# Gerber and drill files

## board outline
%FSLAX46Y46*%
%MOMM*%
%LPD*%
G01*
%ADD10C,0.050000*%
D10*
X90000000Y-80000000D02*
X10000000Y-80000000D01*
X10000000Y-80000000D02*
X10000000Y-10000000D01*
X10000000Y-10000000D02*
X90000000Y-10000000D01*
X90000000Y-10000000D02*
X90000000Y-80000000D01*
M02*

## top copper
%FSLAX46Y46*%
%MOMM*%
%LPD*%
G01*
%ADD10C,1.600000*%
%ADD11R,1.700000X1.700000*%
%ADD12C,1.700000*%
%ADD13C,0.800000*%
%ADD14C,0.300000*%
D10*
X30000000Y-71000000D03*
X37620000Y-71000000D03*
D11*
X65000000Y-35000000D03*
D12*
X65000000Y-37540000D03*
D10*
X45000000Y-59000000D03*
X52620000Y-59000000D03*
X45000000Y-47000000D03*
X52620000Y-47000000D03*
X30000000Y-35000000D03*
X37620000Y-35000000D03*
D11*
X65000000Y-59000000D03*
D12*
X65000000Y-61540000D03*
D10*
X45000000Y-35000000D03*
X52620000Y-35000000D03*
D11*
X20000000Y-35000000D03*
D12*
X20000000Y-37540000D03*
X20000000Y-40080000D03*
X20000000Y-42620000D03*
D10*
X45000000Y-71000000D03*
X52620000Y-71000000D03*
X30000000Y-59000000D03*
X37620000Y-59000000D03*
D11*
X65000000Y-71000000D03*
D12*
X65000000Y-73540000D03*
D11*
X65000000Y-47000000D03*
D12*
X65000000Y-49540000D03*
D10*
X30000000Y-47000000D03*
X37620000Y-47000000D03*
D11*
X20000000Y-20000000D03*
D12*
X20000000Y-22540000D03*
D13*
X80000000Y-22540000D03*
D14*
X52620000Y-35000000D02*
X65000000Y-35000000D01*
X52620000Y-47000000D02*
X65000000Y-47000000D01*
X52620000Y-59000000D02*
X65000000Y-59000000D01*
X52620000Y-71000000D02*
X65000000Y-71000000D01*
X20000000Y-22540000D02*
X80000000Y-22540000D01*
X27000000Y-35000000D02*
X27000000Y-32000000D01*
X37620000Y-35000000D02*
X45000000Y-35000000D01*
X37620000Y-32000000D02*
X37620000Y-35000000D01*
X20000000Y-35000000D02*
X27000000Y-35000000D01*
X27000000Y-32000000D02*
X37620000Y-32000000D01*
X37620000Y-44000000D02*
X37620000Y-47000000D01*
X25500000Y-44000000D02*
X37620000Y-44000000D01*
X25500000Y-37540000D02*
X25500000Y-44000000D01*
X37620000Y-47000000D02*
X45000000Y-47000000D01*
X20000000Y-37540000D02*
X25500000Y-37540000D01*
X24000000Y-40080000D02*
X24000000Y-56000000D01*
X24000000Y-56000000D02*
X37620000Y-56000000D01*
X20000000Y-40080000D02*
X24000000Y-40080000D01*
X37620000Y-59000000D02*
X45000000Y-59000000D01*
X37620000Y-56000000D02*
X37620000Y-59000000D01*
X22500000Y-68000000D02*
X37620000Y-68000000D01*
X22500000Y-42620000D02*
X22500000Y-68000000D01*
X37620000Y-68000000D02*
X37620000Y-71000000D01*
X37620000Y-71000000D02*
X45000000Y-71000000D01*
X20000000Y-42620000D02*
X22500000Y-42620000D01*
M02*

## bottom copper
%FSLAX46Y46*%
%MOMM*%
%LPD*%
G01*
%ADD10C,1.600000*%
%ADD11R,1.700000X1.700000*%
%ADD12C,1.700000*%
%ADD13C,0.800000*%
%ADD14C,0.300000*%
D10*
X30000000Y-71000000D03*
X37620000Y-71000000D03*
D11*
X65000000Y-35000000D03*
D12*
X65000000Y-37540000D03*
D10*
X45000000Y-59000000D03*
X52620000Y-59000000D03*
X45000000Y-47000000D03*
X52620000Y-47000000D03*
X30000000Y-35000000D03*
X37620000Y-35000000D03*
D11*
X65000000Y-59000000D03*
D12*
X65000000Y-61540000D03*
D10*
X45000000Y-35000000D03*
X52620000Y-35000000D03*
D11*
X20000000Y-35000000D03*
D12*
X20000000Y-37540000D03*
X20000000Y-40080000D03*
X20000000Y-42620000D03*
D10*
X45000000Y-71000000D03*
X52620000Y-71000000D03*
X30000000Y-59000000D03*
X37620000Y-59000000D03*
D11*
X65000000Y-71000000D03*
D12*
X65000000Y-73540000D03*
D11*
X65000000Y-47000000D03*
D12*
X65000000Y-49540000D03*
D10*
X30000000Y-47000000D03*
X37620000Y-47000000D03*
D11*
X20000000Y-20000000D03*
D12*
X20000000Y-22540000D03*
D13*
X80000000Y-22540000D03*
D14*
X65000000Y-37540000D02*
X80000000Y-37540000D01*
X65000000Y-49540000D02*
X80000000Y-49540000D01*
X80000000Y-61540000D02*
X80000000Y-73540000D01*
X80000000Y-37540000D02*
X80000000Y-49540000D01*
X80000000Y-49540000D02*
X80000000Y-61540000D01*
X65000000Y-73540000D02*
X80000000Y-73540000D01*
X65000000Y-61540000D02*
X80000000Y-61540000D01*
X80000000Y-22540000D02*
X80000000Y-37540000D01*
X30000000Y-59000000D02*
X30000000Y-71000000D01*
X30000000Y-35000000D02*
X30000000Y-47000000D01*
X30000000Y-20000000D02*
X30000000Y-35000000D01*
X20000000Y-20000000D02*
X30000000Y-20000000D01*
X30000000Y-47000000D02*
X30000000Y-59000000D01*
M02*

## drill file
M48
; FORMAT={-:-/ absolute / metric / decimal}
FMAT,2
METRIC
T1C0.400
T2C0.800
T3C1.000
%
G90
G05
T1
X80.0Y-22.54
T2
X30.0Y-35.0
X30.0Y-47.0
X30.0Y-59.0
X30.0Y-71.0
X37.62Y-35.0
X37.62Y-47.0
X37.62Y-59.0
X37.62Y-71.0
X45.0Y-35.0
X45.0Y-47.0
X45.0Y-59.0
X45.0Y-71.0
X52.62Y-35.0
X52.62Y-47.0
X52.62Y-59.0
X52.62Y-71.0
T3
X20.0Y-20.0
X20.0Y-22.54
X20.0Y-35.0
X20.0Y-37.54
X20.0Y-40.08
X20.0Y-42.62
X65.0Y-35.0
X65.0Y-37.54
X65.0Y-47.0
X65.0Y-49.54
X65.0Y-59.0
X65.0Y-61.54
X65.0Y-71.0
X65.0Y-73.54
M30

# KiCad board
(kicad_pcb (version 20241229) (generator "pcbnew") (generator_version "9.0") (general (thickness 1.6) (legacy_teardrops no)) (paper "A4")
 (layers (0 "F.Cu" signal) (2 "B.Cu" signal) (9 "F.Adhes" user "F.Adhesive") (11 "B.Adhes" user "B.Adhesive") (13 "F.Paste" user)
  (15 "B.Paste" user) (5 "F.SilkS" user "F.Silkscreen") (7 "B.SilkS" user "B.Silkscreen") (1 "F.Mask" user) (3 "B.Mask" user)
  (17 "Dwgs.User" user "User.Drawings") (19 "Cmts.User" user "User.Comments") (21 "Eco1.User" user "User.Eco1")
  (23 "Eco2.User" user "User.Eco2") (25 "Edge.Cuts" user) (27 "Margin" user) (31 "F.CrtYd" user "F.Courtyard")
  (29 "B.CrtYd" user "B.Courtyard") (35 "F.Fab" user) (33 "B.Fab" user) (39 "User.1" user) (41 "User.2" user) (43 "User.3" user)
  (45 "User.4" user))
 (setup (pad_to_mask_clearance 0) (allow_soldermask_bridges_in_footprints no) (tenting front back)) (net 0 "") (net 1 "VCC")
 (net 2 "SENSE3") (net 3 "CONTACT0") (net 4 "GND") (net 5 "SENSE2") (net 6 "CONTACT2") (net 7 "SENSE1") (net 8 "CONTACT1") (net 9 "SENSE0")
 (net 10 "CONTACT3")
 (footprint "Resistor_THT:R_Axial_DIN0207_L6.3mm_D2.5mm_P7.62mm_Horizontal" (layer "F.Cu") (at 30 71)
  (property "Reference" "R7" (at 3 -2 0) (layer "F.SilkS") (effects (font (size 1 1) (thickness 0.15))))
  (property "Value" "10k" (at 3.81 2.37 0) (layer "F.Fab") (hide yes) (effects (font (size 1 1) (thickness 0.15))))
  (pad "1" thru_hole circle (at 0 0) (size 1.6 1.6) (drill 0.8) (layers "*.Cu" "*.Mask") (remove_unused_layers no) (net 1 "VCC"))
  (pad "2" thru_hole circle (at 7.62 0) (size 1.6 1.6) (drill 0.8) (layers "*.Cu" "*.Mask") (remove_unused_layers no) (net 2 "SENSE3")))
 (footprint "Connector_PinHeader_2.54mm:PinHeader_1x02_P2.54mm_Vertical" (layer "F.Cu") (at 65 35)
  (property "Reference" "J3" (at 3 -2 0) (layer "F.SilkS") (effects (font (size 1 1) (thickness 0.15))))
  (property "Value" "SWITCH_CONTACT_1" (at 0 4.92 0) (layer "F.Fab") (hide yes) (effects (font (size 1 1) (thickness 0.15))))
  (pad "1" thru_hole rect (at 0 0) (size 1.7 1.7) (drill 1) (layers "*.Cu" "*.Mask") (remove_unused_layers no) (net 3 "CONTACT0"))
  (pad "2" thru_hole circle (at 0 2.54) (size 1.7 1.7) (drill 1) (layers "*.Cu" "*.Mask") (remove_unused_layers no) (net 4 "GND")))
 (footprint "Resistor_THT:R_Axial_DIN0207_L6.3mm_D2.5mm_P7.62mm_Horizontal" (layer "F.Cu") (at 45 59)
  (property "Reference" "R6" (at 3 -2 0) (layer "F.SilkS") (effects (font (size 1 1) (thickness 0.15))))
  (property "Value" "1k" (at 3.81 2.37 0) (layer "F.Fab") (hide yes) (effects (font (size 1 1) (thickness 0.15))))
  (pad "1" thru_hole circle (at 0 0) (size 1.6 1.6) (drill 0.8) (layers "*.Cu" "*.Mask") (remove_unused_layers no) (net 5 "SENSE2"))
  (pad "2" thru_hole circle (at 7.62 0) (size 1.6 1.6) (drill 0.8) (layers "*.Cu" "*.Mask") (remove_unused_layers no) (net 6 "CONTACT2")))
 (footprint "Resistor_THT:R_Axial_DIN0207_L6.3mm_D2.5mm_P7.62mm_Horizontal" (layer "F.Cu") (at 45 47)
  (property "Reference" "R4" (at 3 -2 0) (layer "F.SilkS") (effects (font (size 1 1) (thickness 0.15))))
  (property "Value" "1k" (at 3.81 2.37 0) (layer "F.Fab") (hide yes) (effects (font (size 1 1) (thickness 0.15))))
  (pad "1" thru_hole circle (at 0 0) (size 1.6 1.6) (drill 0.8) (layers "*.Cu" "*.Mask") (remove_unused_layers no) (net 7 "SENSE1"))
  (pad "2" thru_hole circle (at 7.62 0) (size 1.6 1.6) (drill 0.8) (layers "*.Cu" "*.Mask") (remove_unused_layers no) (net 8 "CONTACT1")))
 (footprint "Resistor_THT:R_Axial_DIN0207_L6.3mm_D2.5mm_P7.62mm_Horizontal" (layer "F.Cu") (at 30 35)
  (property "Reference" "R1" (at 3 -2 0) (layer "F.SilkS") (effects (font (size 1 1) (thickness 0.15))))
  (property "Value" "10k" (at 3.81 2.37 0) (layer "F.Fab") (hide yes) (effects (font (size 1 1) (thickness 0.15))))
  (pad "1" thru_hole circle (at 0 0) (size 1.6 1.6) (drill 0.8) (layers "*.Cu" "*.Mask") (remove_unused_layers no) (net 1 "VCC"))
  (pad "2" thru_hole circle (at 7.62 0) (size 1.6 1.6) (drill 0.8) (layers "*.Cu" "*.Mask") (remove_unused_layers no) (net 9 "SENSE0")))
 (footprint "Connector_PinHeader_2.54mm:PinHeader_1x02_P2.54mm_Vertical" (layer "F.Cu") (at 65 59)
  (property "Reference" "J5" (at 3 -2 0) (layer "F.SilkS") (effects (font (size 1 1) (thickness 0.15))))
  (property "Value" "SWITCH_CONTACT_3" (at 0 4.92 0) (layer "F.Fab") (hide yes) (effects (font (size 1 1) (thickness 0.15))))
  (pad "1" thru_hole rect (at 0 0) (size 1.7 1.7) (drill 1) (layers "*.Cu" "*.Mask") (remove_unused_layers no) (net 6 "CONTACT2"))
  (pad "2" thru_hole circle (at 0 2.54) (size 1.7 1.7) (drill 1) (layers "*.Cu" "*.Mask") (remove_unused_layers no) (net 4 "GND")))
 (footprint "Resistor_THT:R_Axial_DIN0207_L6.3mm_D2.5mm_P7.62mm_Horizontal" (layer "F.Cu") (at 45 35)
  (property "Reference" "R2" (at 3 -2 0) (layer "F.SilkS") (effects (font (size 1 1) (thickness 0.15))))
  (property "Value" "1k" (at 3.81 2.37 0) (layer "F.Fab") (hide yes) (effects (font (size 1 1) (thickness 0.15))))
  (pad "1" thru_hole circle (at 0 0) (size 1.6 1.6) (drill 0.8) (layers "*.Cu" "*.Mask") (remove_unused_layers no) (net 9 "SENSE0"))
  (pad "2" thru_hole circle (at 7.62 0) (size 1.6 1.6) (drill 0.8) (layers "*.Cu" "*.Mask") (remove_unused_layers no) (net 3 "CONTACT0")))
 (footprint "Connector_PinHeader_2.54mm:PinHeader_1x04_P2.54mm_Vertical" (layer "F.Cu") (at 20 35)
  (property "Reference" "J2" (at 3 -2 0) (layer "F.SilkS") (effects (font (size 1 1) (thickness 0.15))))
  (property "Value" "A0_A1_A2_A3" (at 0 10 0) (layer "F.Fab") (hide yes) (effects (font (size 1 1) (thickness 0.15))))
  (pad "1" thru_hole rect (at 0 0) (size 1.7 1.7) (drill 1) (layers "*.Cu" "*.Mask") (remove_unused_layers no) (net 9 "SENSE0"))
  (pad "2" thru_hole circle (at 0 2.54) (size 1.7 1.7) (drill 1) (layers "*.Cu" "*.Mask") (remove_unused_layers no) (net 7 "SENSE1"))
  (pad "3" thru_hole circle (at 0 5.08) (size 1.7 1.7) (drill 1) (layers "*.Cu" "*.Mask") (remove_unused_layers no) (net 5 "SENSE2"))
  (pad "4" thru_hole circle (at 0 7.62) (size 1.7 1.7) (drill 1) (layers "*.Cu" "*.Mask") (remove_unused_layers no) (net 2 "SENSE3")))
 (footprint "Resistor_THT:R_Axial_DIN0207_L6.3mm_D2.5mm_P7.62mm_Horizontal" (layer "F.Cu") (at 45 71)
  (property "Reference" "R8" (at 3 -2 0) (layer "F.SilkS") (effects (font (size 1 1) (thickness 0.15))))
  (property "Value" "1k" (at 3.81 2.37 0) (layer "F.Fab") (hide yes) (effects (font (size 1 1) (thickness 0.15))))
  (pad "1" thru_hole circle (at 0 0) (size 1.6 1.6) (drill 0.8) (layers "*.Cu" "*.Mask") (remove_unused_layers no) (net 2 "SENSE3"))
  (pad "2" thru_hole circle (at 7.62 0) (size 1.6 1.6) (drill 0.8) (layers "*.Cu" "*.Mask") (remove_unused_layers no) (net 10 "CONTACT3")))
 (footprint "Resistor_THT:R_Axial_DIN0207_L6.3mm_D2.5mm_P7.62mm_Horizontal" (layer "F.Cu") (at 30 59)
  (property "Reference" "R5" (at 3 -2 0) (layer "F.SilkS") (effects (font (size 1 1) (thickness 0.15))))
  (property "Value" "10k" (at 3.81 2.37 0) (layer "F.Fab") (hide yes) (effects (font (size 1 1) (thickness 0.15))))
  (pad "1" thru_hole circle (at 0 0) (size 1.6 1.6) (drill 0.8) (layers "*.Cu" "*.Mask") (remove_unused_layers no) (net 1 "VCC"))
  (pad "2" thru_hole circle (at 7.62 0) (size 1.6 1.6) (drill 0.8) (layers "*.Cu" "*.Mask") (remove_unused_layers no) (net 5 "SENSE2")))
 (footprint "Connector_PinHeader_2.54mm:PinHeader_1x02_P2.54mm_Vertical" (layer "F.Cu") (at 65 71)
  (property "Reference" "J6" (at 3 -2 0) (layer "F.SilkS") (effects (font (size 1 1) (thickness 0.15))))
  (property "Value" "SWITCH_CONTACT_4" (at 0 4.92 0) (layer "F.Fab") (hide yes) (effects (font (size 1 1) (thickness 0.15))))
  (pad "1" thru_hole rect (at 0 0) (size 1.7 1.7) (drill 1) (layers "*.Cu" "*.Mask") (remove_unused_layers no) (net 10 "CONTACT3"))
  (pad "2" thru_hole circle (at 0 2.54) (size 1.7 1.7) (drill 1) (layers "*.Cu" "*.Mask") (remove_unused_layers no) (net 4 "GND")))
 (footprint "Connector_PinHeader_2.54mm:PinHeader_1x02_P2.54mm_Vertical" (layer "F.Cu") (at 65 47)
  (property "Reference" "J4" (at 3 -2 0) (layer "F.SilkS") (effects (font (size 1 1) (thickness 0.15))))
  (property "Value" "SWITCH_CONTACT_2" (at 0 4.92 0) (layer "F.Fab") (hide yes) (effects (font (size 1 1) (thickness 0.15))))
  (pad "1" thru_hole rect (at 0 0) (size 1.7 1.7) (drill 1) (layers "*.Cu" "*.Mask") (remove_unused_layers no) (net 8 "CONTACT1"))
  (pad "2" thru_hole circle (at 0 2.54) (size 1.7 1.7) (drill 1) (layers "*.Cu" "*.Mask") (remove_unused_layers no) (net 4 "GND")))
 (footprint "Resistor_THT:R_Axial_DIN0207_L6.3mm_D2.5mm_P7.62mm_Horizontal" (layer "F.Cu") (at 30 47)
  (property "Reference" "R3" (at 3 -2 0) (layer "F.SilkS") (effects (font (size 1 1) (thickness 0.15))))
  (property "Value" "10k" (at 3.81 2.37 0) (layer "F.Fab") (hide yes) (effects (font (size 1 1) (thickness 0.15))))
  (pad "1" thru_hole circle (at 0 0) (size 1.6 1.6) (drill 0.8) (layers "*.Cu" "*.Mask") (remove_unused_layers no) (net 1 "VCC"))
  (pad "2" thru_hole circle (at 7.62 0) (size 1.6 1.6) (drill 0.8) (layers "*.Cu" "*.Mask") (remove_unused_layers no) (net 7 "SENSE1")))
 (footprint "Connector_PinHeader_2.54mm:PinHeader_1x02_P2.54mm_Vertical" (layer "F.Cu") (at 20 20)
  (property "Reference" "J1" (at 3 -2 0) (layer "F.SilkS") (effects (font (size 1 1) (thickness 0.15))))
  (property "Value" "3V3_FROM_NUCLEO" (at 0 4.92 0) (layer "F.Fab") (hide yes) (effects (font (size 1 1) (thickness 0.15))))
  (pad "1" thru_hole rect (at 0 0) (size 1.7 1.7) (drill 1) (layers "*.Cu" "*.Mask") (remove_unused_layers no) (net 1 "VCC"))
  (pad "2" thru_hole circle (at 0 2.54) (size 1.7 1.7) (drill 1) (layers "*.Cu" "*.Mask") (remove_unused_layers no) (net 4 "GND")))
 (gr_line (start 90 80) (end 10 80) (stroke (width 0.05) (type default)) (layer "Edge.Cuts"))
 (gr_line (start 10 80) (end 10 10) (stroke (width 0.05) (type default)) (layer "Edge.Cuts"))
 (gr_line (start 10 10) (end 90 10) (stroke (width 0.05) (type default)) (layer "Edge.Cuts"))
 (gr_line (start 90 10) (end 90 80) (stroke (width 0.05) (type default)) (layer "Edge.Cuts"))
 (segment (start 52.62 35) (end 65 35) (width 0.3) (layer "F.Cu") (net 3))
 (segment (start 52.62 47) (end 65 47) (width 0.3) (layer "F.Cu") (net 8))
 (segment (start 52.62 59) (end 65 59) (width 0.3) (layer "F.Cu") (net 6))
 (segment (start 52.62 71) (end 65 71) (width 0.3) (layer "F.Cu") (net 10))
 (segment (start 20 22.54) (end 80 22.54) (width 0.3) (layer "F.Cu") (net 4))
 (via (at 80 22.54) (size 0.8) (drill 0.4) (layers "F.Cu" "B.Cu") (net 4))
 (segment (start 65 37.54) (end 80 37.54) (width 0.3) (layer "B.Cu") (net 4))
 (segment (start 65 49.54) (end 80 49.54) (width 0.3) (layer "B.Cu") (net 4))
 (segment (start 80 61.54) (end 80 73.54) (width 0.3) (layer "B.Cu") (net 4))
 (segment (start 80 37.54) (end 80 49.54) (width 0.3) (layer "B.Cu") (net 4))
 (segment (start 80 49.54) (end 80 61.54) (width 0.3) (layer "B.Cu") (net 4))
 (segment (start 65 73.54) (end 80 73.54) (width 0.3) (layer "B.Cu") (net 4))
 (segment (start 65 61.54) (end 80 61.54) (width 0.3) (layer "B.Cu") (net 4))
 (segment (start 80 22.54) (end 80 37.54) (width 0.3) (layer "B.Cu") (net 4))
 (segment (start 27 35) (end 27 32) (width 0.3) (layer "F.Cu") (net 9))
 (segment (start 37.62 35) (end 45 35) (width 0.3) (layer "F.Cu") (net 9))
 (segment (start 37.62 32) (end 37.62 35) (width 0.3) (layer "F.Cu") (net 9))
 (segment (start 20 35) (end 27 35) (width 0.3) (layer "F.Cu") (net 9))
 (segment (start 27 32) (end 37.62 32) (width 0.3) (layer "F.Cu") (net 9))
 (segment (start 37.62 44) (end 37.62 47) (width 0.3) (layer "F.Cu") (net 7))
 (segment (start 25.5 44) (end 37.62 44) (width 0.3) (layer "F.Cu") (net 7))
 (segment (start 25.5 37.54) (end 25.5 44) (width 0.3) (layer "F.Cu") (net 7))
 (segment (start 37.62 47) (end 45 47) (width 0.3) (layer "F.Cu") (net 7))
 (segment (start 20 37.54) (end 25.5 37.54) (width 0.3) (layer "F.Cu") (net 7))
 (segment (start 24 40.08) (end 24 56) (width 0.3) (layer "F.Cu") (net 5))
 (segment (start 24 56) (end 37.62 56) (width 0.3) (layer "F.Cu") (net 5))
 (segment (start 20 40.08) (end 24 40.08) (width 0.3) (layer "F.Cu") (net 5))
 (segment (start 37.62 59) (end 45 59) (width 0.3) (layer "F.Cu") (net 5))
 (segment (start 37.62 56) (end 37.62 59) (width 0.3) (layer "F.Cu") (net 5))
 (segment (start 22.5 68) (end 37.62 68) (width 0.3) (layer "F.Cu") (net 2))
 (segment (start 22.5 42.62) (end 22.5 68) (width 0.3) (layer "F.Cu") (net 2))
 (segment (start 37.62 68) (end 37.62 71) (width 0.3) (layer "F.Cu") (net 2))
 (segment (start 37.62 71) (end 45 71) (width 0.3) (layer "F.Cu") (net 2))
 (segment (start 20 42.62) (end 22.5 42.62) (width 0.3) (layer "F.Cu") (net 2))
 (segment (start 30 59) (end 30 71) (width 0.3) (layer "B.Cu") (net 1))
 (segment (start 30 35) (end 30 47) (width 0.3) (layer "B.Cu") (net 1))
 (segment (start 30 20) (end 30 35) (width 0.3) (layer "B.Cu") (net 1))
 (segment (start 20 20) (end 30 20) (width 0.3) (layer "B.Cu") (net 1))
 (segment (start 30 47) (end 30 59) (width 0.3) (layer "B.Cu") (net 1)))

